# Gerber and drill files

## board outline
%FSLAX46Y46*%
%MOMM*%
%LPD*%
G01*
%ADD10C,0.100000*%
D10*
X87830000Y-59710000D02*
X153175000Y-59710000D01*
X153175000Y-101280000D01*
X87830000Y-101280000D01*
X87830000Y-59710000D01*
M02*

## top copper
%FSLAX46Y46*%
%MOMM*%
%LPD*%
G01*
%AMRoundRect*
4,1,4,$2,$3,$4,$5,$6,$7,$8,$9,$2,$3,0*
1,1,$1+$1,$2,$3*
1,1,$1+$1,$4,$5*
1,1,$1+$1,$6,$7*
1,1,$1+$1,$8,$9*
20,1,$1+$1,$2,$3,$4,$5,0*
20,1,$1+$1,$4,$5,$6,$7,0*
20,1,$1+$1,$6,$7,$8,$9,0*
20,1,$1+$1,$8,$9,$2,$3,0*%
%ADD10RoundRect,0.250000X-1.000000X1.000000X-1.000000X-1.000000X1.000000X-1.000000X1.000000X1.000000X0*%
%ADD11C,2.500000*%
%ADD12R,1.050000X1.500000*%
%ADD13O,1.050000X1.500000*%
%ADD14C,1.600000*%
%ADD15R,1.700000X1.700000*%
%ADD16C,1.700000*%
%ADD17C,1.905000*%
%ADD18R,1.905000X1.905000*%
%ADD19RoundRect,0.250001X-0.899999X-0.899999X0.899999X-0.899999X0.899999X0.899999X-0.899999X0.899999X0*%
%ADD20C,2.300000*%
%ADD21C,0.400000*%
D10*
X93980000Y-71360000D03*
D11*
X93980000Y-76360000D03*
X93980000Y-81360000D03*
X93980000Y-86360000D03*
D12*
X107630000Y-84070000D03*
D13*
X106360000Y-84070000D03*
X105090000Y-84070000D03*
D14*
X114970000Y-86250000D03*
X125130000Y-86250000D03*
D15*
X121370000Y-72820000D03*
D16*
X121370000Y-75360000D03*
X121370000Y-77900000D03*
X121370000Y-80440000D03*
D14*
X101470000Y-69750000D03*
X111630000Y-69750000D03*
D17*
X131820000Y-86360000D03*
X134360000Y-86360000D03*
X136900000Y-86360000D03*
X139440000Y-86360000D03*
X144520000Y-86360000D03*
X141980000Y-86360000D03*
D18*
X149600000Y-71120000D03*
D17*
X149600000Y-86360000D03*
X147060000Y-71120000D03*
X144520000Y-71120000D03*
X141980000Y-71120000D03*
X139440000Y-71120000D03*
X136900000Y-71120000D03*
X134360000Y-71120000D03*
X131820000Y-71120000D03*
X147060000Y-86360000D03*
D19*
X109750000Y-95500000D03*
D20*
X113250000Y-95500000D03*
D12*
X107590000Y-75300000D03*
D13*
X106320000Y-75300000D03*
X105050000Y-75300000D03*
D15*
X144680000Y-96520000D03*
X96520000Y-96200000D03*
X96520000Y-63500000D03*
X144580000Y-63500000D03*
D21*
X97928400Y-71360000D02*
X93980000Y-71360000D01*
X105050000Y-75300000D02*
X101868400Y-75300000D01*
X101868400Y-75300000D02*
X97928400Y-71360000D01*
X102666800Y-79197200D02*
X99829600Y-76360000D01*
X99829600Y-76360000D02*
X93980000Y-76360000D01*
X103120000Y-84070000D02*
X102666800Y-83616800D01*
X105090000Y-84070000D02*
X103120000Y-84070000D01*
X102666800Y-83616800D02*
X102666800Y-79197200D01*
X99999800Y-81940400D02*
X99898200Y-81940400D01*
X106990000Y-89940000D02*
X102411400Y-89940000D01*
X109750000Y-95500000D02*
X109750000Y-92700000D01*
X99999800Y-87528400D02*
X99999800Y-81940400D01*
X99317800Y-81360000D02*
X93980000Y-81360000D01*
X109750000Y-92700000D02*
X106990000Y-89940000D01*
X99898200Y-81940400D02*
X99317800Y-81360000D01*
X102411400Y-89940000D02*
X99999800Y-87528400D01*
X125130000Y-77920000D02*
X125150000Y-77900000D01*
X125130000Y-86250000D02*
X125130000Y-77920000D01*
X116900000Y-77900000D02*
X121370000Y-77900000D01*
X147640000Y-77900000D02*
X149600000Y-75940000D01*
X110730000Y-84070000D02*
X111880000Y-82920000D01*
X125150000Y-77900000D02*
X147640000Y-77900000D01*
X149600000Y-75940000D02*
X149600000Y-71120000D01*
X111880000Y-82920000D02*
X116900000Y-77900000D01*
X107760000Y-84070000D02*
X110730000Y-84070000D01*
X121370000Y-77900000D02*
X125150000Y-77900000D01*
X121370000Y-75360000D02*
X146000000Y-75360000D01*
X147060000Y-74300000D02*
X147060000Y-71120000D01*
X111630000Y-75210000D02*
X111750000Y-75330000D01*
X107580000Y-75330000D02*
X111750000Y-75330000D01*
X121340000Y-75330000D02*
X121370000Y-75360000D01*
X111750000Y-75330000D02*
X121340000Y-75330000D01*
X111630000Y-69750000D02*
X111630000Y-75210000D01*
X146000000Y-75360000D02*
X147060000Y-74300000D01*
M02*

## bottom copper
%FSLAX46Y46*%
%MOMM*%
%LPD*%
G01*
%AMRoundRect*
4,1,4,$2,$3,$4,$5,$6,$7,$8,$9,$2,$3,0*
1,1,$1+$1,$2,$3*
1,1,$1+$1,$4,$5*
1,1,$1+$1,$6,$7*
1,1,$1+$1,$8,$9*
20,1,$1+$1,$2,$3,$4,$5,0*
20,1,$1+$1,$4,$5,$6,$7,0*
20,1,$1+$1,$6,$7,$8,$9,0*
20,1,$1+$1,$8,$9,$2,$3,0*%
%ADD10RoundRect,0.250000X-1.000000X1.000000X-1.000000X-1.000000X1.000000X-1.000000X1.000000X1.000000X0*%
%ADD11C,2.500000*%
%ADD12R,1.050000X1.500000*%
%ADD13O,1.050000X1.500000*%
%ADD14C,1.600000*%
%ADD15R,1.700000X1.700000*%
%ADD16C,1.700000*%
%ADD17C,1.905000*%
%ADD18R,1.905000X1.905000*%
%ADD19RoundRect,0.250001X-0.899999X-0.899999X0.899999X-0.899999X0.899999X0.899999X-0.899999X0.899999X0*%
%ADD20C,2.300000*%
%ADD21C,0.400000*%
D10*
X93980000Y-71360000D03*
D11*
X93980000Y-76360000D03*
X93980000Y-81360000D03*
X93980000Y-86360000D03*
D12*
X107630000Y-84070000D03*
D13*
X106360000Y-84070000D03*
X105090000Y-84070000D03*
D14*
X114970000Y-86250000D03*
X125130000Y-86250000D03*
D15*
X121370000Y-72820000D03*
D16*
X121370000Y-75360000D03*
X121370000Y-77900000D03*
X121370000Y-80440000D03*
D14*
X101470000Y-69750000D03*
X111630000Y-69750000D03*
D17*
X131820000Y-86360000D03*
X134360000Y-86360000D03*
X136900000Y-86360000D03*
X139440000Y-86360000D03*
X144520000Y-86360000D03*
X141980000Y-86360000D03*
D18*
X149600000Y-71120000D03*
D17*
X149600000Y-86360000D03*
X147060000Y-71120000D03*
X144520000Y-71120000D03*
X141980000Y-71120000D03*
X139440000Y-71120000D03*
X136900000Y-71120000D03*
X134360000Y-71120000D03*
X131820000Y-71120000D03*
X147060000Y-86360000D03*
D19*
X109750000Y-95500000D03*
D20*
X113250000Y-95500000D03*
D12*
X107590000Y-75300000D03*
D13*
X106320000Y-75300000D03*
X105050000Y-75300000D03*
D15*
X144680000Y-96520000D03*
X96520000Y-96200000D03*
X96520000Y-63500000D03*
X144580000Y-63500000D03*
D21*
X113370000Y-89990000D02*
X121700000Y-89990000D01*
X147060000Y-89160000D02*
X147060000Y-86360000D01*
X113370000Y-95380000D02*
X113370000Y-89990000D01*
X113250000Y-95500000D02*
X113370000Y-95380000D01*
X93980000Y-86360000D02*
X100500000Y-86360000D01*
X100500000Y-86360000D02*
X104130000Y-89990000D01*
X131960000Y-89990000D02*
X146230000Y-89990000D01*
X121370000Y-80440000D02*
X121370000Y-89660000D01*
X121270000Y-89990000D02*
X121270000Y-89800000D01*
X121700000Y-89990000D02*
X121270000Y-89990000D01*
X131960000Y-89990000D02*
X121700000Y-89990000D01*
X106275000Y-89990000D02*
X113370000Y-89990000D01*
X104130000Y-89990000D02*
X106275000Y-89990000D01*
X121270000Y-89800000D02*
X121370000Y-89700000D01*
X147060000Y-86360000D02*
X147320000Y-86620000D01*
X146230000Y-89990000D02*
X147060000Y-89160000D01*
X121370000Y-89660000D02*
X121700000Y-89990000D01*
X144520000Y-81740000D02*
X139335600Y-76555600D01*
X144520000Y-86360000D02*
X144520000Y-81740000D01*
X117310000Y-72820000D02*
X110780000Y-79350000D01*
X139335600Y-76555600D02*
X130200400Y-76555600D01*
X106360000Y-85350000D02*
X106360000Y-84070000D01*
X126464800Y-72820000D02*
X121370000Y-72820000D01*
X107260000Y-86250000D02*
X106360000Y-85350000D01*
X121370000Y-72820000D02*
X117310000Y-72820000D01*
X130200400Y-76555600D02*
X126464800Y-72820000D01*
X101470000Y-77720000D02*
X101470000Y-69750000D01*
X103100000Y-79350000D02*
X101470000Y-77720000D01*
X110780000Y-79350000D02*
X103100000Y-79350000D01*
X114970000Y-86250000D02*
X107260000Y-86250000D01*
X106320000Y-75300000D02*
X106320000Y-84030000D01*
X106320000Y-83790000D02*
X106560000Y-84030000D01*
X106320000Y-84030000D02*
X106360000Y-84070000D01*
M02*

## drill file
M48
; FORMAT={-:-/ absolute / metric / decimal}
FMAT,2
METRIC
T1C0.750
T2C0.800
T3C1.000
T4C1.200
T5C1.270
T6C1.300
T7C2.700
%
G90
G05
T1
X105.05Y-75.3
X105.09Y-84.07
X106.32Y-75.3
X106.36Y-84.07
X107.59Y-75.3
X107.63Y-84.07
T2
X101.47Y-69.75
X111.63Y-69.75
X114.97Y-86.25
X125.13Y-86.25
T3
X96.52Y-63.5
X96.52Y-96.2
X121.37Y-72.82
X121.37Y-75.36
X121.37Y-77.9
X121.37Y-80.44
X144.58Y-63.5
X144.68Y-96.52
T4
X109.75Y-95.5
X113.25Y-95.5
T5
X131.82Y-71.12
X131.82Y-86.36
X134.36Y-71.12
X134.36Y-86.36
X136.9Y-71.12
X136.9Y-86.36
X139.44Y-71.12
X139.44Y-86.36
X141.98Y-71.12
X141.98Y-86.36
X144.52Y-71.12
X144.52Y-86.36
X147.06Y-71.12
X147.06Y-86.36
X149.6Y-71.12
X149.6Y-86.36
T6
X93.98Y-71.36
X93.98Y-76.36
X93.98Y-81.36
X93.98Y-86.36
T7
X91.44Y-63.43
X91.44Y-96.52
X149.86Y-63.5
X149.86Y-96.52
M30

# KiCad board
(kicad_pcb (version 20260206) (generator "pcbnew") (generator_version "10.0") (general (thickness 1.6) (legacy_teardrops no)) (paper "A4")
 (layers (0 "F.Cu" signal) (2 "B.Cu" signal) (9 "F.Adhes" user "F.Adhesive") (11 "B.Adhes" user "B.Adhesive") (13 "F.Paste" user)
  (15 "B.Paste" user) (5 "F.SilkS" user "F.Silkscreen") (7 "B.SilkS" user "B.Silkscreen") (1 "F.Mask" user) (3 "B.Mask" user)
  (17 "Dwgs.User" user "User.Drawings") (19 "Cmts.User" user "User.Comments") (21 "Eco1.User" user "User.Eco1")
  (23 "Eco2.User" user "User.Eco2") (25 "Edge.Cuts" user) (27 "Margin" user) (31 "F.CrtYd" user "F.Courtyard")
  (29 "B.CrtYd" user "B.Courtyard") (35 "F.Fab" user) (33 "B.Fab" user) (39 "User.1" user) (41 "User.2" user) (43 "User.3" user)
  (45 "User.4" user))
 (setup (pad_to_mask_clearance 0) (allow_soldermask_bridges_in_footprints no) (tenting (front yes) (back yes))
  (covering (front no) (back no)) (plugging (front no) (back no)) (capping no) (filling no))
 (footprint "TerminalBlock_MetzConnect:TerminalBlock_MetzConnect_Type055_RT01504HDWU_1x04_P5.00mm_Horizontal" (layer "F.Cu")
  (at 93.98 71.36 -90)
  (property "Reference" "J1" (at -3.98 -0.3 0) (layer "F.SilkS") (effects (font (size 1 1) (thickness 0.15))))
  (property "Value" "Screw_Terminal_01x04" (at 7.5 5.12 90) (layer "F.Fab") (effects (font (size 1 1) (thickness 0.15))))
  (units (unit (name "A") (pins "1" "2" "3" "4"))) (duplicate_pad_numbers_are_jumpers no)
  (pad "1" thru_hole roundrect (at 0 0 270) (size 2.5 2.5) (drill 1.3) (layers "*.Cu" "*.Mask") (remove_unused_layers no)
   (roundrect_rratio 0.1) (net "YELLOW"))
  (pad "2" thru_hole circle (at 5 0 270) (size 2.5 2.5) (drill 1.3) (layers "*.Cu" "*.Mask") (remove_unused_layers no) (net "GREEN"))
  (pad "3" thru_hole circle (at 10 0 270) (size 2.5 2.5) (drill 1.3) (layers "*.Cu" "*.Mask") (remove_unused_layers no) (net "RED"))
  (pad "4" thru_hole circle (at 15 0 270) (size 2.5 2.5) (drill 1.3) (layers "*.Cu" "*.Mask") (remove_unused_layers no) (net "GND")))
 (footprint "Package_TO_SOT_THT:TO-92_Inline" (layer "F.Cu") (at 107.63 84.07 180)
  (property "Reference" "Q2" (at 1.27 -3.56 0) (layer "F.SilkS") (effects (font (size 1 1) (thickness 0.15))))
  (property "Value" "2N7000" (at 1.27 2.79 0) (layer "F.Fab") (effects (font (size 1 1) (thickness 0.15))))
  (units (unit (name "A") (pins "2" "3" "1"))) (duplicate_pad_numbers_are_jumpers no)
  (pad "1" thru_hole rect (at 0 0 180) (size 1.05 1.5) (drill 0.75) (layers "*.Cu" "*.Mask") (remove_unused_layers no) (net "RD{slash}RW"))
  (pad "2" thru_hole oval (at 1.27 0 180) (size 1.05 1.5) (drill 0.75) (layers "*.Cu" "*.Mask") (remove_unused_layers no) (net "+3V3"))
  (pad "3" thru_hole oval (at 2.54 0 180) (size 1.05 1.5) (drill 0.75) (layers "*.Cu" "*.Mask") (remove_unused_layers no) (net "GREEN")))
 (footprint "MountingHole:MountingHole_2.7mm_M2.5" (layer "F.Cu") (at 149.86 63.5)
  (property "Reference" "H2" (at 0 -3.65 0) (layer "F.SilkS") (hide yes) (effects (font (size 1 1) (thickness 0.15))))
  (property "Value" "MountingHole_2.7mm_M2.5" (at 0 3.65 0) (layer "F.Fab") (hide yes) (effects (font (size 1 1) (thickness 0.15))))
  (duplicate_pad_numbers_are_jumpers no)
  (pad "" np_thru_hole circle (at 0 0) (size 2.7 2.7) (drill 2.7) (layers "*.Cu" "*.Mask")))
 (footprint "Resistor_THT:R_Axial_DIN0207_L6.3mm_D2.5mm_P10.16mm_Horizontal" (layer "F.Cu") (at 114.97 86.25)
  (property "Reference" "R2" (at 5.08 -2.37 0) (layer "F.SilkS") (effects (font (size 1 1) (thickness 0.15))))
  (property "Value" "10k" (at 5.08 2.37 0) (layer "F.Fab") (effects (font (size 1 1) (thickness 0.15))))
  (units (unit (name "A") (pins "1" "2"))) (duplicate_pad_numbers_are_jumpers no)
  (pad "1" thru_hole circle (at 0 0) (size 1.6 1.6) (drill 0.8) (layers "*.Cu" "*.Mask") (remove_unused_layers no) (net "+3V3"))
  (pad "2" thru_hole circle (at 10.16 0) (size 1.6 1.6) (drill 0.8) (layers "*.Cu" "*.Mask") (remove_unused_layers no) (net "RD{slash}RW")))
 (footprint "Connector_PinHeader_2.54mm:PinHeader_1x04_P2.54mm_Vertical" (layer "F.Cu") (at 121.37 72.82)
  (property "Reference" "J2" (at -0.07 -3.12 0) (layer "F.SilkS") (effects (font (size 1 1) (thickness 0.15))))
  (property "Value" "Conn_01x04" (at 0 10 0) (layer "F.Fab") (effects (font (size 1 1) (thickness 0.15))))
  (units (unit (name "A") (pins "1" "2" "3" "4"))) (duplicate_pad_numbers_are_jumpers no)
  (pad "1" thru_hole rect (at 0 0) (size 1.7 1.7) (drill 1) (layers "*.Cu" "*.Mask") (remove_unused_layers no) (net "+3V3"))
  (pad "2" thru_hole circle (at 0 2.54) (size 1.7 1.7) (drill 1) (layers "*.Cu" "*.Mask") (remove_unused_layers no) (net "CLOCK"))
  (pad "3" thru_hole circle (at 0 5.08) (size 1.7 1.7) (drill 1) (layers "*.Cu" "*.Mask") (remove_unused_layers no) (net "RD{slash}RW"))
  (pad "4" thru_hole circle (at 0 7.62) (size 1.7 1.7) (drill 1) (layers "*.Cu" "*.Mask") (remove_unused_layers no) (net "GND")))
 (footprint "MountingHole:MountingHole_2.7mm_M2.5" (layer "F.Cu") (at 91.44 96.52)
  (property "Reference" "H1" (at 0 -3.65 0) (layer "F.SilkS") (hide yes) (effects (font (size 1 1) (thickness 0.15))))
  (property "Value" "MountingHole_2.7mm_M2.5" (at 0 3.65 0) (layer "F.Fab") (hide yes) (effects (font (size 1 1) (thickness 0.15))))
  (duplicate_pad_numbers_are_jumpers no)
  (pad "" np_thru_hole circle (at 0 0) (size 2.7 2.7) (drill 2.7) (layers "*.Cu" "*.Mask")))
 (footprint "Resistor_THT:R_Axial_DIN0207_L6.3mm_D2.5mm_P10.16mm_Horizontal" (layer "F.Cu") (at 101.47 69.75)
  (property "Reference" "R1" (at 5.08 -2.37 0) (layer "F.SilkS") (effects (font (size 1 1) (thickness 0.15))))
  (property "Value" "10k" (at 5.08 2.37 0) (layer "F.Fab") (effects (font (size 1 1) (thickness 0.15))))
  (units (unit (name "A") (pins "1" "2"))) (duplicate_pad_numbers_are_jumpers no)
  (pad "1" thru_hole circle (at 0 0) (size 1.6 1.6) (drill 0.8) (layers "*.Cu" "*.Mask") (remove_unused_layers no) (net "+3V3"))
  (pad "2" thru_hole circle (at 10.16 0) (size 1.6 1.6) (drill 0.8) (layers "*.Cu" "*.Mask") (remove_unused_layers no) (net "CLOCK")))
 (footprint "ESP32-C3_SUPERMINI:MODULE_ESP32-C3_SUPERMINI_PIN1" (layer "F.Cu") (at 139.7 78.74 -90)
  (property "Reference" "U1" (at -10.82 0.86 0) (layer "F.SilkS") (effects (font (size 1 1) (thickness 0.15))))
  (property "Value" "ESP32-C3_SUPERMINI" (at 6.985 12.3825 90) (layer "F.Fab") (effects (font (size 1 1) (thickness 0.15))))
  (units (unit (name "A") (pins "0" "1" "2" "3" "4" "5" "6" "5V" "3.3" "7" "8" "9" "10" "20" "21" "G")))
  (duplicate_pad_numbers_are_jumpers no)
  (pad "0" thru_hole circle (at 7.62 7.88 270) (size 1.905 1.905) (drill 1.27) (layers "*.Cu" "*.Mask") (remove_unused_layers no)
   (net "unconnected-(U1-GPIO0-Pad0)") (solder_mask_margin 0.102))
  (pad "1" thru_hole circle (at 7.62 5.34 270) (size 1.905 1.905) (drill 1.27) (layers "*.Cu" "*.Mask") (remove_unused_layers no)
   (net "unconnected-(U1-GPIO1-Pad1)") (solder_mask_margin 0.102))
  (pad "2" thru_hole circle (at 7.62 2.8 270) (size 1.905 1.905) (drill 1.27) (layers "*.Cu" "*.Mask") (remove_unused_layers no)
   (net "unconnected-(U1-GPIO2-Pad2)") (solder_mask_margin 0.102))
  (pad "3" thru_hole circle (at 7.62 0.26 270) (size 1.905 1.905) (drill 1.27) (layers "*.Cu" "*.Mask") (remove_unused_layers no)
   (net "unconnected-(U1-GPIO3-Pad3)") (solder_mask_margin 0.102))
  (pad "3.3" thru_hole circle (at 7.62 -4.82 270) (size 1.905 1.905) (drill 1.27) (layers "*.Cu" "*.Mask") (remove_unused_layers no)
   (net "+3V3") (solder_mask_margin 0.102))
  (pad "4" thru_hole circle (at 7.62 -2.28 270) (size 1.905 1.905) (drill 1.27) (layers "*.Cu" "*.Mask") (remove_unused_layers no)
   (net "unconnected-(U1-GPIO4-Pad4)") (solder_mask_margin 0.102))
  (pad "5" thru_hole rect (at -7.62 -9.9 270) (size 1.905 1.905) (drill 1.27) (layers "*.Cu" "*.Mask") (remove_unused_layers no)
   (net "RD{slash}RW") (solder_mask_margin 0.102))
  (pad "5V" thru_hole circle (at 7.62 -9.9 270) (size 1.905 1.905) (drill 1.27) (layers "*.Cu" "*.Mask") (remove_unused_layers no)
   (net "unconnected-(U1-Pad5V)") (solder_mask_margin 0.102))
  (pad "6" thru_hole circle (at -7.62 -7.36 270) (size 1.905 1.905) (drill 1.27) (layers "*.Cu" "*.Mask") (remove_unused_layers no)
   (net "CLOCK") (solder_mask_margin 0.102))
  (pad "7" thru_hole circle (at -7.62 -4.82 270) (size 1.905 1.905) (drill 1.27) (layers "*.Cu" "*.Mask") (remove_unused_layers no)
   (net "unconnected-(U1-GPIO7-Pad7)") (solder_mask_margin 0.102))
  (pad "8" thru_hole circle (at -7.62 -2.28 270) (size 1.905 1.905) (drill 1.27) (layers "*.Cu" "*.Mask") (remove_unused_layers no)
   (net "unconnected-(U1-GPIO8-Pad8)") (solder_mask_margin 0.102))
  (pad "9" thru_hole circle (at -7.62 0.26 270) (size 1.905 1.905) (drill 1.27) (layers "*.Cu" "*.Mask") (remove_unused_layers no)
   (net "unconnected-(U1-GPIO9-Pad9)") (solder_mask_margin 0.102))
  (pad "10" thru_hole circle (at -7.62 2.8 270) (size 1.905 1.905) (drill 1.27) (layers "*.Cu" "*.Mask") (remove_unused_layers no)
   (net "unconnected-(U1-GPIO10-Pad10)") (solder_mask_margin 0.102))
  (pad "20" thru_hole circle (at -7.62 5.34 270) (size 1.905 1.905) (drill 1.27) (layers "*.Cu" "*.Mask") (remove_unused_layers no)
   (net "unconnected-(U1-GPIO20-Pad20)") (solder_mask_margin 0.102))
  (pad "21" thru_hole circle (at -7.62 7.88 270) (size 1.905 1.905) (drill 1.27) (layers "*.Cu" "*.Mask") (remove_unused_layers no)
   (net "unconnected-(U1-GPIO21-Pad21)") (solder_mask_margin 0.102))
  (pad "G" thru_hole circle (at 7.62 -7.36 270) (size 1.905 1.905) (drill 1.27) (layers "*.Cu" "*.Mask") (remove_unused_layers no)
   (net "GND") (solder_mask_margin 0.102)))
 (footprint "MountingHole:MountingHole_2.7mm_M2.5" (layer "F.Cu") (at 91.44 63.43)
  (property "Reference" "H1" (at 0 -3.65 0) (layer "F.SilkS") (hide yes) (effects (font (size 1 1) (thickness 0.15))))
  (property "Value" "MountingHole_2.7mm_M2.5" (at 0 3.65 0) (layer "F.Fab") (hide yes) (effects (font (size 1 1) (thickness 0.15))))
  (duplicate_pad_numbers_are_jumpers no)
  (pad "" np_thru_hole circle (at 0 0) (size 2.7 2.7) (drill 2.7) (layers "*.Cu" "*.Mask")))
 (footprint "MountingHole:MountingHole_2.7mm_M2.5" (layer "F.Cu") (at 149.86 96.52)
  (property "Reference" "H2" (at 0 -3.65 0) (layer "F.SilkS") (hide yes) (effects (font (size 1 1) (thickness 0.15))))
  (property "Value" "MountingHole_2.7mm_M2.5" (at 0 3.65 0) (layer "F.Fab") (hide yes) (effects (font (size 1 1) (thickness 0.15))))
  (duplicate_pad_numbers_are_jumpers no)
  (pad "" np_thru_hole circle (at 0 0) (size 2.7 2.7) (drill 2.7) (layers "*.Cu" "*.Mask")))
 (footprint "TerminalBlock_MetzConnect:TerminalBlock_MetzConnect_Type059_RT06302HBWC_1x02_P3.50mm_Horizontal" (layer "F.Cu")
  (at 109.75 95.5)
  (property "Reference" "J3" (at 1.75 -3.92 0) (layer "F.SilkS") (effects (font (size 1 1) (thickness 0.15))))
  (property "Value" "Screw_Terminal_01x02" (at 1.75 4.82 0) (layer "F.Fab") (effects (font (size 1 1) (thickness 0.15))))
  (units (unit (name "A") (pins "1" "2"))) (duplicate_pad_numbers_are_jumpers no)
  (pad "1" thru_hole roundrect (at 0 0) (size 2.3 2.3) (drill 1.2) (layers "*.Cu" "*.Mask") (remove_unused_layers no)
   (roundrect_rratio 0.108696) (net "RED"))
  (pad "2" thru_hole circle (at 3.5 0) (size 2.3 2.3) (drill 1.2) (layers "*.Cu" "*.Mask") (remove_unused_layers no) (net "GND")))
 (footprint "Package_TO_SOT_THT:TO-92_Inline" (layer "F.Cu") (at 107.59 75.3 180)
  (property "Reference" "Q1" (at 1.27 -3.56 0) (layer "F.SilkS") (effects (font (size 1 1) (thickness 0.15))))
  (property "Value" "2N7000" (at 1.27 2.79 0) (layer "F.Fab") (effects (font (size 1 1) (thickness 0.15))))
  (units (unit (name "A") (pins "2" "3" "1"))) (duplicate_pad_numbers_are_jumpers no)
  (pad "1" thru_hole rect (at 0 0 180) (size 1.05 1.5) (drill 0.75) (layers "*.Cu" "*.Mask") (remove_unused_layers no) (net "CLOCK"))
  (pad "2" thru_hole oval (at 1.27 0 180) (size 1.05 1.5) (drill 0.75) (layers "*.Cu" "*.Mask") (remove_unused_layers no) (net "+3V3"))
  (pad "3" thru_hole oval (at 2.54 0 180) (size 1.05 1.5) (drill 0.75) (layers "*.Cu" "*.Mask") (remove_unused_layers no) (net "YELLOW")))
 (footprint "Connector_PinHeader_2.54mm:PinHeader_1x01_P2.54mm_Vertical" (layer "B.Cu") (at 144.68 96.52)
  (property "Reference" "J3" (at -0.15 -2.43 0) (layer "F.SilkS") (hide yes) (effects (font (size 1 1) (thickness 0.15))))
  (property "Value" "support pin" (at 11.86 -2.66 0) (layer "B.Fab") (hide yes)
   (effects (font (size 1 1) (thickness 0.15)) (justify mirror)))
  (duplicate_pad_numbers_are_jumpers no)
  (pad "1" thru_hole rect (at 0 0) (size 1.7 1.7) (drill 1) (layers "*.Cu" "*.Mask") (remove_unused_layers no)))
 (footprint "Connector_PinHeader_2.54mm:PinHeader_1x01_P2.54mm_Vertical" (layer "B.Cu") (at 96.52 96.2)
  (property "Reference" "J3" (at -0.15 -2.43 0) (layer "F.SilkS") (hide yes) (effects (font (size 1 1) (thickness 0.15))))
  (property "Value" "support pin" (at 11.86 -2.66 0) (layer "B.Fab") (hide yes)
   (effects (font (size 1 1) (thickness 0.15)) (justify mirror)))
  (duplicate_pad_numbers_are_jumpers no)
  (pad "1" thru_hole rect (at 0 0) (size 1.7 1.7) (drill 1) (layers "*.Cu" "*.Mask") (remove_unused_layers no)))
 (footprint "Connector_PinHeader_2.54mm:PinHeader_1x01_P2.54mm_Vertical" (layer "B.Cu") (at 96.52 63.5)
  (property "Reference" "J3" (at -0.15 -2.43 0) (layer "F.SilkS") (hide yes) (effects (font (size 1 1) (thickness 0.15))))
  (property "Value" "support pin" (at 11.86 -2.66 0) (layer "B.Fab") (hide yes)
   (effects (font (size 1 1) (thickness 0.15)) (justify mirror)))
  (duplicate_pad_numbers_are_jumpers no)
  (pad "1" thru_hole rect (at 0 0) (size 1.7 1.7) (drill 1) (layers "*.Cu" "*.Mask") (remove_unused_layers no)))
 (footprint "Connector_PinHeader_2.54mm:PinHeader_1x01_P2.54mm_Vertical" (layer "B.Cu") (at 144.58 63.5)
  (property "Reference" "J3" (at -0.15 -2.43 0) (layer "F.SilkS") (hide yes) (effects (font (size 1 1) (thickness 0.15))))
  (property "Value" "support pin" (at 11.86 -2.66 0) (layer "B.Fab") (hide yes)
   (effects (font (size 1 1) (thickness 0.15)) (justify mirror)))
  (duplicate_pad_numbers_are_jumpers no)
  (pad "1" thru_hole rect (at 0 0) (size 1.7 1.7) (drill 1) (layers "*.Cu" "*.Mask") (remove_unused_layers no)))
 (gr_rect (start 87.83 59.71) (end 153.175 101.28) (stroke (width 0.1) (type default)) (fill no) (layer "Edge.Cuts"))
 (segment (start 97.9284 71.36) (end 93.98 71.36) (width 0.4) (layer "F.Cu") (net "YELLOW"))
 (segment (start 105.05 75.3) (end 101.8684 75.3) (width 0.4) (layer "F.Cu") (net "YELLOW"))
 (segment (start 101.8684 75.3) (end 97.9284 71.36) (width 0.4) (layer "F.Cu") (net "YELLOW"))
 (segment (start 102.6668 79.1972) (end 99.8296 76.36) (width 0.4) (layer "F.Cu") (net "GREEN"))
 (segment (start 99.8296 76.36) (end 93.98 76.36) (width 0.4) (layer "F.Cu") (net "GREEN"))
 (segment (start 103.12 84.07) (end 102.6668 83.6168) (width 0.4) (layer "F.Cu") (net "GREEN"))
 (segment (start 105.09 84.07) (end 103.12 84.07) (width 0.4) (layer "F.Cu") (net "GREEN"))
 (segment (start 102.6668 83.6168) (end 102.6668 79.1972) (width 0.4) (layer "F.Cu") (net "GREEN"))
 (segment (start 99.9998 81.9404) (end 99.8982 81.9404) (width 0.4) (layer "F.Cu") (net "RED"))
 (segment (start 106.99 89.94) (end 102.4114 89.94) (width 0.4) (layer "F.Cu") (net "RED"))
 (segment (start 109.75 95.5) (end 109.75 92.7) (width 0.4) (layer "F.Cu") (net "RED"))
 (segment (start 99.9998 87.5284) (end 99.9998 81.9404) (width 0.4) (layer "F.Cu") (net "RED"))
 (segment (start 99.3178 81.36) (end 93.98 81.36) (width 0.4) (layer "F.Cu") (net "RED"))
 (segment (start 109.75 92.7) (end 106.99 89.94) (width 0.4) (layer "F.Cu") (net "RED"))
 (segment (start 99.8982 81.9404) (end 99.3178 81.36) (width 0.4) (layer "F.Cu") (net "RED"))
 (segment (start 102.4114 89.94) (end 99.9998 87.5284) (width 0.4) (layer "F.Cu") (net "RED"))
 (segment (start 113.37 89.99) (end 121.7 89.99) (width 0.4) (layer "B.Cu") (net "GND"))
 (segment (start 147.06 89.16) (end 147.06 86.36) (width 0.4) (layer "B.Cu") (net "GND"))
 (segment (start 113.37 95.38) (end 113.37 89.99) (width 0.4) (layer "B.Cu") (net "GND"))
 (segment (start 113.25 95.5) (end 113.37 95.38) (width 0.4) (layer "B.Cu") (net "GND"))
 (segment (start 93.98 86.36) (end 100.5 86.36) (width 0.4) (layer "B.Cu") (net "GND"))
 (segment (start 100.5 86.36) (end 104.13 89.99) (width 0.4) (layer "B.Cu") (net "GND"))
 (segment (start 131.96 89.99) (end 146.23 89.99) (width 0.4) (layer "B.Cu") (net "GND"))
 (segment (start 121.37 80.44) (end 121.37 89.66) (width 0.4) (layer "B.Cu") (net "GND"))
 (segment (start 121.27 89.99) (end 121.27 89.8) (width 0.4) (layer "B.Cu") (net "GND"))
 (segment (start 121.7 89.99) (end 121.27 89.99) (width 0.4) (layer "B.Cu") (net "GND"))
 (segment (start 131.96 89.99) (end 121.7 89.99) (width 0.4) (layer "B.Cu") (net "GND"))
 (segment (start 106.275 89.99) (end 113.37 89.99) (width 0.4) (layer "B.Cu") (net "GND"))
 (segment (start 104.13 89.99) (end 106.275 89.99) (width 0.4) (layer "B.Cu") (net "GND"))
 (segment (start 121.27 89.8) (end 121.37 89.7) (width 0.4) (layer "B.Cu") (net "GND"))
 (segment (start 147.06 86.36) (end 147.32 86.62) (width 0.4) (layer "B.Cu") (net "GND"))
 (segment (start 146.23 89.99) (end 147.06 89.16) (width 0.4) (layer "B.Cu") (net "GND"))
 (segment (start 121.37 89.66) (end 121.7 89.99) (width 0.4) (layer "B.Cu") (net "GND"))
 (segment (start 125.13 77.92) (end 125.15 77.9) (width 0.4) (layer "F.Cu") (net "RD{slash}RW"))
 (segment (start 125.13 86.25) (end 125.13 77.92) (width 0.4) (layer "F.Cu") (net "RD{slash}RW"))
 (segment (start 116.9 77.9) (end 121.37 77.9) (width 0.4) (layer "F.Cu") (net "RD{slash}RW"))
 (segment (start 147.64 77.9) (end 149.6 75.94) (width 0.4) (layer "F.Cu") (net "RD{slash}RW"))
 (segment (start 110.73 84.07) (end 111.88 82.92) (width 0.4) (layer "F.Cu") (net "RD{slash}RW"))
 (segment (start 125.15 77.9) (end 147.64 77.9) (width 0.4) (layer "F.Cu") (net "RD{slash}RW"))
 (segment (start 149.6 75.94) (end 149.6 71.12) (width 0.4) (layer "F.Cu") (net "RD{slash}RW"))
 (segment (start 111.88 82.92) (end 116.9 77.9) (width 0.4) (layer "F.Cu") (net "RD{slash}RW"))
 (segment (start 107.76 84.07) (end 110.73 84.07) (width 0.4) (layer "F.Cu") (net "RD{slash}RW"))
 (segment (start 121.37 77.9) (end 125.15 77.9) (width 0.4) (layer "F.Cu") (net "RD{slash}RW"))
 (segment (start 144.52 81.74) (end 139.3356 76.5556) (width 0.4) (layer "B.Cu") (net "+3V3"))
 (segment (start 144.52 86.36) (end 144.52 81.74) (width 0.4) (layer "B.Cu") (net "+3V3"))
 (segment (start 117.31 72.82) (end 110.78 79.35) (width 0.4) (layer "B.Cu") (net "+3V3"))
 (segment (start 139.3356 76.5556) (end 130.2004 76.5556) (width 0.4) (layer "B.Cu") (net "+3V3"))
 (segment (start 106.36 85.35) (end 106.36 84.07) (width 0.4) (layer "B.Cu") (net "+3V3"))
 (segment (start 126.4648 72.82) (end 121.37 72.82) (width 0.4) (layer "B.Cu") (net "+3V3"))
 (segment (start 107.26 86.25) (end 106.36 85.35) (width 0.4) (layer "B.Cu") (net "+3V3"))
 (segment (start 121.37 72.82) (end 117.31 72.82) (width 0.4) (layer "B.Cu") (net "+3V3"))
 (segment (start 130.2004 76.5556) (end 126.4648 72.82) (width 0.4) (layer "B.Cu") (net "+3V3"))
 (segment (start 101.47 77.72) (end 101.47 69.75) (width 0.4) (layer "B.Cu") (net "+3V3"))
 (segment (start 103.1 79.35) (end 101.47 77.72) (width 0.4) (layer "B.Cu") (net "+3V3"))
 (segment (start 110.78 79.35) (end 103.1 79.35) (width 0.4) (layer "B.Cu") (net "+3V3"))
 (segment (start 114.97 86.25) (end 107.26 86.25) (width 0.4) (layer "B.Cu") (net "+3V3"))
 (segment (start 106.32 75.3) (end 106.32 84.03) (width 0.4) (layer "B.Cu") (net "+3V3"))
 (segment (start 106.32 83.79) (end 106.56 84.03) (width 0.4) (layer "B.Cu") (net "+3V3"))
 (segment (start 106.32 84.03) (end 106.36 84.07) (width 0.4) (layer "B.Cu") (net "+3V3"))
 (segment (start 121.37 75.36) (end 146 75.36) (width 0.4) (layer "F.Cu") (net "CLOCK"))
 (segment (start 147.06 74.3) (end 147.06 71.12) (width 0.4) (layer "F.Cu") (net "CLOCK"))
 (segment (start 111.63 75.21) (end 111.75 75.33) (width 0.4) (layer "F.Cu") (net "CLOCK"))
 (segment (start 107.58 75.33) (end 111.75 75.33) (width 0.4) (layer "F.Cu") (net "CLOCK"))
 (segment (start 121.34 75.33) (end 121.37 75.36) (width 0.4) (layer "F.Cu") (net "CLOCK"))
 (segment (start 111.75 75.33) (end 121.34 75.33) (width 0.4) (layer "F.Cu") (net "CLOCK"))
 (segment (start 111.63 69.75) (end 111.63 75.21) (width 0.4) (layer "F.Cu") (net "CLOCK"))
 (segment (start 146 75.36) (end 147.06 74.3) (width 0.4) (layer "F.Cu") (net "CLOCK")))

